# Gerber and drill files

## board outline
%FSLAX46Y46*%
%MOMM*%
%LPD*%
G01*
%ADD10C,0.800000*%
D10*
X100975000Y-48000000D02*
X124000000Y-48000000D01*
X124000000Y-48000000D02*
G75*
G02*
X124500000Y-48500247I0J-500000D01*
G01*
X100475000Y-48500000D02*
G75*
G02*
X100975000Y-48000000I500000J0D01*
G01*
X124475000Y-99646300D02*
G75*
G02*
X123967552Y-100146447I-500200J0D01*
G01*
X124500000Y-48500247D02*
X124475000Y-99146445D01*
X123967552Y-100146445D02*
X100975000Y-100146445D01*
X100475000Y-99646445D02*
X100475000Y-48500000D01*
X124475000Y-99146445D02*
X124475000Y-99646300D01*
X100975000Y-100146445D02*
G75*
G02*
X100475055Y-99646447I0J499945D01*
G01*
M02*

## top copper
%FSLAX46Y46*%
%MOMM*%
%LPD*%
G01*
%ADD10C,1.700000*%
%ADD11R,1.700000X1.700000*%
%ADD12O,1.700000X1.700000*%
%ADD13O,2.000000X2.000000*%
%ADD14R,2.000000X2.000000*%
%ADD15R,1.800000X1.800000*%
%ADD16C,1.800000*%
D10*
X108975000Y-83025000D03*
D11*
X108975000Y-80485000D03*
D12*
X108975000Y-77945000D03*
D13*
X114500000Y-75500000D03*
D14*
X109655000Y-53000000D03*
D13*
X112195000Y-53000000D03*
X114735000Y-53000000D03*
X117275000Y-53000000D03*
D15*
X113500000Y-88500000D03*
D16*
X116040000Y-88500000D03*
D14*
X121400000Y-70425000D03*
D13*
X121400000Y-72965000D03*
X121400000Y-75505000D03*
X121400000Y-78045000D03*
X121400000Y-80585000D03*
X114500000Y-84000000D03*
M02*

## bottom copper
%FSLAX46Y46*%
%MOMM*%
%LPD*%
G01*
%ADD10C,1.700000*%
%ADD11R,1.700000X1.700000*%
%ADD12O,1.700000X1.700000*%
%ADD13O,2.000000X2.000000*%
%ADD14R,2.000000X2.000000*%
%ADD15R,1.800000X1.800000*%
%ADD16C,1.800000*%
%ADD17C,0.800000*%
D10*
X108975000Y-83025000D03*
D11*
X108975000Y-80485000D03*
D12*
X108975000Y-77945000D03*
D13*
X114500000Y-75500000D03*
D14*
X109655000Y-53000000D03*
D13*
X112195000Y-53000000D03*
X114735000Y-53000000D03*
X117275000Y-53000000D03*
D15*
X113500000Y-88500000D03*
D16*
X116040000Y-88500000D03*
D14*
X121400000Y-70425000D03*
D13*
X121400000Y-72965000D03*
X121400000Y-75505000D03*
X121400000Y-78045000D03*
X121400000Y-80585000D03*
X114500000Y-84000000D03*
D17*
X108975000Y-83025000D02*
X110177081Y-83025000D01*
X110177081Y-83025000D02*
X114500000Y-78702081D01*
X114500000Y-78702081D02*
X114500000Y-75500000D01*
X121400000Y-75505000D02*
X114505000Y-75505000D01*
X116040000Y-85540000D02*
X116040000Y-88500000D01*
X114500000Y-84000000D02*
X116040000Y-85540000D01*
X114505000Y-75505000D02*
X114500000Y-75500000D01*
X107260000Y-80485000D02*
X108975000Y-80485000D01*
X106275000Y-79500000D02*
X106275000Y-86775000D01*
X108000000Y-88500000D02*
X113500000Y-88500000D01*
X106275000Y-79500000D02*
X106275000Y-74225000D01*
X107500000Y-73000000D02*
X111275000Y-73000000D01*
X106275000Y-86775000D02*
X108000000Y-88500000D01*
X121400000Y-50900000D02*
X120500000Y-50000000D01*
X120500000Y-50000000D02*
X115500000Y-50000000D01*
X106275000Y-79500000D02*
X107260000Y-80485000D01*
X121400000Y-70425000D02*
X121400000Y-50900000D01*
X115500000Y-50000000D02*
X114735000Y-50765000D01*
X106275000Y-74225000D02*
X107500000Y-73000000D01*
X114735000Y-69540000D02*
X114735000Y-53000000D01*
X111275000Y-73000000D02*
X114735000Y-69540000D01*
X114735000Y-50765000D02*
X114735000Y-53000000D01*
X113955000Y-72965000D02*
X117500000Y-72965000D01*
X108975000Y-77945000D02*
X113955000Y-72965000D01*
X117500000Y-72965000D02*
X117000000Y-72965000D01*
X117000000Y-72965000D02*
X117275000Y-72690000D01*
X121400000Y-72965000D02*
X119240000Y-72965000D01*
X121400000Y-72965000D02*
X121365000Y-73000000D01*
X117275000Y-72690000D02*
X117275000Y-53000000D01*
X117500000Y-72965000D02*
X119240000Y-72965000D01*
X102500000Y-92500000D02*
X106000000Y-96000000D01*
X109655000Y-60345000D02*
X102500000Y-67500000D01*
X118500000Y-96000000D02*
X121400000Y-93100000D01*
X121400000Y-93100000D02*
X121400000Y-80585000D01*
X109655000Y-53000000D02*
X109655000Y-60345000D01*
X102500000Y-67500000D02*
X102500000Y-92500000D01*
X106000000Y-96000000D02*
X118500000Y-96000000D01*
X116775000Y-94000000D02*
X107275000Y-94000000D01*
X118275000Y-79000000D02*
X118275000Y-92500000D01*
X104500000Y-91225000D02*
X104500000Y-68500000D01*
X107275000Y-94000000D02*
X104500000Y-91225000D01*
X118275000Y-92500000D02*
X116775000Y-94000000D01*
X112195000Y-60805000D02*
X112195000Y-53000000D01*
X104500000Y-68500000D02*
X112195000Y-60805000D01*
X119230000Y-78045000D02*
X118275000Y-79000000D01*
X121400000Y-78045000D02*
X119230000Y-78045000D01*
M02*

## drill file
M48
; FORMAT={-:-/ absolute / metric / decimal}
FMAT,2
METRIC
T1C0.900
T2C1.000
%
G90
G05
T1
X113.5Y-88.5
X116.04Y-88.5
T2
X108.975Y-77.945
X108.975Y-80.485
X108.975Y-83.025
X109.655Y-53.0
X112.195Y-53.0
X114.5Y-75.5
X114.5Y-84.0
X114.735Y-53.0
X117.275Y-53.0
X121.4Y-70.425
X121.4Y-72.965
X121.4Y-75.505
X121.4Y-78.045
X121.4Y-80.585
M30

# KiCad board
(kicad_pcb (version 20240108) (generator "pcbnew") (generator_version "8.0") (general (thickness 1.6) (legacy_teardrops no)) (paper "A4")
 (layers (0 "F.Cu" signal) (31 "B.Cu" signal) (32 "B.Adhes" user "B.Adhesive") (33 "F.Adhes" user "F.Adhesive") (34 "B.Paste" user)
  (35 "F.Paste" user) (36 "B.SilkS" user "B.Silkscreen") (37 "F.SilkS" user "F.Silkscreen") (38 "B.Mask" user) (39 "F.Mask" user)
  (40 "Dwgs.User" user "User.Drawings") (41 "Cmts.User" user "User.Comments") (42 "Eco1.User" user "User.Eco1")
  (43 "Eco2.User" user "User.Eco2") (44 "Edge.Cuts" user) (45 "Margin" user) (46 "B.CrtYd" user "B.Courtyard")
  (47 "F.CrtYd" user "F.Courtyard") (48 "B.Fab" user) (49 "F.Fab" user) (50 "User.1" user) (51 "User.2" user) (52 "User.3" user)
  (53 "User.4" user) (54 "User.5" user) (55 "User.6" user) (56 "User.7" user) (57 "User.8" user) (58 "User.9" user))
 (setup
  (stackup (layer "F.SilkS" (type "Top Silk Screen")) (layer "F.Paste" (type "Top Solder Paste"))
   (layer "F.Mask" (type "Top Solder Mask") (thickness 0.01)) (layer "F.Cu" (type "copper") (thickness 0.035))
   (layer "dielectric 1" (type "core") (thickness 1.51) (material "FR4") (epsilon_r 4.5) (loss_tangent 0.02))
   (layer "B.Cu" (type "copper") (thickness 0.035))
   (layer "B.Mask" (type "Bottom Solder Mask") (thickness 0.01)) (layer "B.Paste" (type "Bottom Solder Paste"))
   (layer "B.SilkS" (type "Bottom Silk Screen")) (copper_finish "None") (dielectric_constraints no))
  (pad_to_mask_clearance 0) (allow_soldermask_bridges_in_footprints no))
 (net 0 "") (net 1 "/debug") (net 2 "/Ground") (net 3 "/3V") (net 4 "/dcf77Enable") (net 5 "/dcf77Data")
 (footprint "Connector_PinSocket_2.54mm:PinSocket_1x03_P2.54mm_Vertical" (layer "F.Cu") (at 108.975 83.025 180)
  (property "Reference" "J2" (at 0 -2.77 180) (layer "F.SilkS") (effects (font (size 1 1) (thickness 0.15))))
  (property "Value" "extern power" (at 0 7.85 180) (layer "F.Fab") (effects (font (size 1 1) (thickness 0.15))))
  (pad "1" thru_hole circle (at 0 0 180) (size 1.7 1.7) (drill 1) (layers "*.Cu" "*.Mask") (remove_unused_layers no) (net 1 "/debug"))
  (pad "2" thru_hole rect (at 0 2.54 180) (size 1.7 1.7) (drill 1) (layers "*.Cu" "*.Mask") (remove_unused_layers no) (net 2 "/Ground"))
  (pad "3" thru_hole oval (at 0 5.08 180) (size 1.7 1.7) (drill 1) (layers "*.Cu" "*.Mask") (remove_unused_layers no) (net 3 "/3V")))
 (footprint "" (layer "F.Cu") (at 114.5 75.5 90)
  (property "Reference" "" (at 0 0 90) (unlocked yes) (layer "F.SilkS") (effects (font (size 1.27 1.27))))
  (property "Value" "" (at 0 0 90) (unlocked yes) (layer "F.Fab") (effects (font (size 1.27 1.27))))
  (pad "3" thru_hole oval (at 0 0 90) (size 2 2) (drill 1) (layers "*.Cu" "*.Mask") (remove_unused_layers no) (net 1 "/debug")))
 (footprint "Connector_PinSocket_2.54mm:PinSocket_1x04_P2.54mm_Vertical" (layer "F.Cu") (at 109.655 53 90)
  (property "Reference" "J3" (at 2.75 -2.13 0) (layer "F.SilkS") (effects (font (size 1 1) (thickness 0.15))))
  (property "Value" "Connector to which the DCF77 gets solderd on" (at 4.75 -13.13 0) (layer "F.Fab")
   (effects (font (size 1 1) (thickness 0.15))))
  (pad "1" thru_hole rect (at 0 0 90) (size 2 2) (drill 1) (layers "*.Cu" "*.Mask") (remove_unused_layers no) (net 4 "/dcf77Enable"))
  (pad "2" thru_hole oval (at 0 2.54 90) (size 2 2) (drill 1) (layers "*.Cu" "*.Mask") (remove_unused_layers no) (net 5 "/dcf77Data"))
  (pad "3" thru_hole oval (at 0 5.08 90) (size 2 2) (drill 1) (layers "*.Cu" "*.Mask") (remove_unused_layers no) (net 2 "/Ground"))
  (pad "4" thru_hole oval (at 0 7.62 90) (size 2 2) (drill 1) (layers "*.Cu" "*.Mask") (remove_unused_layers no) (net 3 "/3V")))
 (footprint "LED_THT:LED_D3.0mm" (layer "F.Cu") (at 113.5 88.5)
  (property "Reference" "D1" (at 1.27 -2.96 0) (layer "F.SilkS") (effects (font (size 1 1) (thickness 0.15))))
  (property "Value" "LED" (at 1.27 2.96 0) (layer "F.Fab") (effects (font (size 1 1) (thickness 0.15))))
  (pad "1" thru_hole rect (at 0 0) (size 1.8 1.8) (drill 0.9) (layers "*.Cu" "*.Mask") (remove_unused_layers no) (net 2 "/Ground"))
  (pad "2" thru_hole circle (at 2.54 0) (size 1.8 1.8) (drill 0.9) (layers "*.Cu" "*.Mask") (remove_unused_layers no) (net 1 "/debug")))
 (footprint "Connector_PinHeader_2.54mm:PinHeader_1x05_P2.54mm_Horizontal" (layer "F.Cu") (at 121.4 70.425)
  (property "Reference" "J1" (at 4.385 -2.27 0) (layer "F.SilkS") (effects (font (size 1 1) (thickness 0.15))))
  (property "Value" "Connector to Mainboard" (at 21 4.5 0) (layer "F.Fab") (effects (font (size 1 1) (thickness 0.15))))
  (pad "1" thru_hole rect (at 0 0) (size 2 2) (drill 1) (layers "*.Cu" "*.Mask") (remove_unused_layers no) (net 2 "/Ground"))
  (pad "2" thru_hole oval (at 0 2.54) (size 2 2) (drill 1) (layers "*.Cu" "*.Mask") (remove_unused_layers no) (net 3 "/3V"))
  (pad "3" thru_hole oval (at 0 5.08) (size 2 2) (drill 1) (layers "*.Cu" "*.Mask") (remove_unused_layers no) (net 1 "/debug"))
  (pad "4" thru_hole oval (at 0 7.62) (size 2 2) (drill 1) (layers "*.Cu" "*.Mask") (remove_unused_layers no) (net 5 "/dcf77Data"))
  (pad "5" thru_hole oval (at 0 10.16) (size 2 2) (drill 1) (layers "*.Cu" "*.Mask") (remove_unused_layers no) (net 4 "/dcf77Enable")))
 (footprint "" (layer "F.Cu") (at 114.5 84 90)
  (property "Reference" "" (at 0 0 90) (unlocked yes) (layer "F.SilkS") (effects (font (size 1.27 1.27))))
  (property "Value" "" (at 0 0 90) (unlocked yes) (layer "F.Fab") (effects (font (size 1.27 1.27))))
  (pad "3" thru_hole oval (at 0 0 90) (size 2 2) (drill 1) (layers "*.Cu" "*.Mask") (remove_unused_layers no) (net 1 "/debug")))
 (gr_line (start 100.975 48) (end 124 48) (stroke (width 0.8) (type default)) (layer "Edge.Cuts"))
 (gr_arc (start 124 48) (mid 124.353553 48.146447) (end 124.5 48.500247) (stroke (width 0.8) (type default)) (layer "Edge.Cuts"))
 (gr_arc (start 100.475 48.5) (mid 100.621447 48.146447) (end 100.975 48) (stroke (width 0.8) (type default)) (layer "Edge.Cuts"))
 (gr_arc (start 124.475 99.6463) (mid 124.328537 99.99997) (end 123.967552 100.146445) (stroke (width 0.8) (type default))
  (layer "Edge.Cuts"))
 (gr_line (start 124.5 48.500247) (end 124.475 99.146445) (stroke (width 0.8) (type default)) (layer "Edge.Cuts"))
 (gr_line (start 123.967552 100.146445) (end 100.975 100.146445) (stroke (width 0.8) (type default)) (layer "Edge.Cuts"))
 (gr_line (start 100.475 99.646445) (end 100.475 48.5) (stroke (width 0.8) (type default)) (layer "Edge.Cuts"))
 (gr_line (start 124.475 99.146445) (end 124.475 99.6463) (stroke (width 0.8) (type default)) (layer "Edge.Cuts"))
 (gr_arc (start 100.975 100.146445) (mid 100.621429 100.000003) (end 100.474998 99.646447) (stroke (width 0.8) (type default))
  (layer "Edge.Cuts"))
 (segment (start 108.975 83.025) (end 110.177081 83.025) (width 0.8) (layer "B.Cu") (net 1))
 (segment (start 110.177081 83.025) (end 114.5 78.702081) (width 0.8) (layer "B.Cu") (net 1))
 (segment (start 114.5 78.702081) (end 114.5 75.5) (width 0.8) (layer "B.Cu") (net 1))
 (segment (start 121.4 75.505) (end 114.505 75.505) (width 0.8) (layer "B.Cu") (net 1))
 (segment (start 116.04 85.54) (end 116.04 88.5) (width 0.8) (layer "B.Cu") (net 1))
 (segment (start 114.5 84) (end 116.04 85.54) (width 0.8) (layer "B.Cu") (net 1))
 (segment (start 114.505 75.505) (end 114.5 75.5) (width 0.8) (layer "B.Cu") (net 1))
 (segment (start 107.26 80.485) (end 108.975 80.485) (width 0.8) (layer "B.Cu") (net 2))
 (segment (start 106.275 79.5) (end 106.275 86.775) (width 0.8) (layer "B.Cu") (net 2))
 (segment (start 108 88.5) (end 113.5 88.5) (width 0.8) (layer "B.Cu") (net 2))
 (segment (start 106.275 79.5) (end 106.275 74.225) (width 0.8) (layer "B.Cu") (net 2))
 (segment (start 107.5 73) (end 111.275 73) (width 0.8) (layer "B.Cu") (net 2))
 (segment (start 106.275 86.775) (end 108 88.5) (width 0.8) (layer "B.Cu") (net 2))
 (segment (start 121.4 50.9) (end 120.5 50) (width 0.8) (layer "B.Cu") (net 2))
 (segment (start 120.5 50) (end 115.5 50) (width 0.8) (layer "B.Cu") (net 2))
 (segment (start 106.275 79.5) (end 107.26 80.485) (width 0.8) (layer "B.Cu") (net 2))
 (segment (start 121.4 70.425) (end 121.4 50.9) (width 0.8) (layer "B.Cu") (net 2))
 (segment (start 115.5 50) (end 114.735 50.765) (width 0.8) (layer "B.Cu") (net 2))
 (segment (start 106.275 74.225) (end 107.5 73) (width 0.8) (layer "B.Cu") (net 2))
 (segment (start 114.735 69.54) (end 114.735 53) (width 0.8) (layer "B.Cu") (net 2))
 (segment (start 111.275 73) (end 114.735 69.54) (width 0.8) (layer "B.Cu") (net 2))
 (segment (start 114.735 50.765) (end 114.735 53) (width 0.8) (layer "B.Cu") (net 2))
 (segment (start 113.955 72.965) (end 117.5 72.965) (width 0.8) (layer "B.Cu") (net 3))
 (segment (start 108.975 77.945) (end 113.955 72.965) (width 0.8) (layer "B.Cu") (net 3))
 (segment (start 117.5 72.965) (end 117 72.965) (width 0.8) (layer "B.Cu") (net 3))
 (segment (start 117 72.965) (end 117.275 72.69) (width 0.8) (layer "B.Cu") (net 3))
 (segment (start 121.4 72.965) (end 119.24 72.965) (width 0.8) (layer "B.Cu") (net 3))
 (segment (start 121.4 72.965) (end 121.365 73) (width 0.8) (layer "B.Cu") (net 3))
 (segment (start 117.275 72.69) (end 117.275 53) (width 0.8) (layer "B.Cu") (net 3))
 (segment (start 117.5 72.965) (end 119.24 72.965) (width 0.8) (layer "B.Cu") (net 3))
 (segment (start 102.5 92.5) (end 106 96) (width 0.8) (layer "B.Cu") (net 4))
 (segment (start 109.655 60.345) (end 102.5 67.5) (width 0.8) (layer "B.Cu") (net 4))
 (segment (start 118.5 96) (end 121.4 93.1) (width 0.8) (layer "B.Cu") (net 4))
 (segment (start 121.4 93.1) (end 121.4 80.585) (width 0.8) (layer "B.Cu") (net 4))
 (segment (start 109.655 53) (end 109.655 60.345) (width 0.8) (layer "B.Cu") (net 4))
 (segment (start 102.5 67.5) (end 102.5 92.5) (width 0.8) (layer "B.Cu") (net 4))
 (segment (start 106 96) (end 118.5 96) (width 0.8) (layer "B.Cu") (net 4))
 (segment (start 116.775 94) (end 107.275 94) (width 0.8) (layer "B.Cu") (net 5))
 (segment (start 118.275 79) (end 118.275 92.5) (width 0.8) (layer "B.Cu") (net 5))
 (segment (start 104.5 91.225) (end 104.5 68.5) (width 0.8) (layer "B.Cu") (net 5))
 (segment (start 107.275 94) (end 104.5 91.225) (width 0.8) (layer "B.Cu") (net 5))
 (segment (start 118.275 92.5) (end 116.775 94) (width 0.8) (layer "B.Cu") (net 5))
 (segment (start 112.195 60.805) (end 112.195 53) (width 0.8) (layer "B.Cu") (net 5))
 (segment (start 104.5 68.5) (end 112.195 60.805) (width 0.8) (layer "B.Cu") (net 5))
 (segment (start 119.23 78.045) (end 118.275 79) (width 0.8) (layer "B.Cu") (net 5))
 (segment (start 121.4 78.045) (end 119.23 78.045) (width 0.8) (layer "B.Cu") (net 5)))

